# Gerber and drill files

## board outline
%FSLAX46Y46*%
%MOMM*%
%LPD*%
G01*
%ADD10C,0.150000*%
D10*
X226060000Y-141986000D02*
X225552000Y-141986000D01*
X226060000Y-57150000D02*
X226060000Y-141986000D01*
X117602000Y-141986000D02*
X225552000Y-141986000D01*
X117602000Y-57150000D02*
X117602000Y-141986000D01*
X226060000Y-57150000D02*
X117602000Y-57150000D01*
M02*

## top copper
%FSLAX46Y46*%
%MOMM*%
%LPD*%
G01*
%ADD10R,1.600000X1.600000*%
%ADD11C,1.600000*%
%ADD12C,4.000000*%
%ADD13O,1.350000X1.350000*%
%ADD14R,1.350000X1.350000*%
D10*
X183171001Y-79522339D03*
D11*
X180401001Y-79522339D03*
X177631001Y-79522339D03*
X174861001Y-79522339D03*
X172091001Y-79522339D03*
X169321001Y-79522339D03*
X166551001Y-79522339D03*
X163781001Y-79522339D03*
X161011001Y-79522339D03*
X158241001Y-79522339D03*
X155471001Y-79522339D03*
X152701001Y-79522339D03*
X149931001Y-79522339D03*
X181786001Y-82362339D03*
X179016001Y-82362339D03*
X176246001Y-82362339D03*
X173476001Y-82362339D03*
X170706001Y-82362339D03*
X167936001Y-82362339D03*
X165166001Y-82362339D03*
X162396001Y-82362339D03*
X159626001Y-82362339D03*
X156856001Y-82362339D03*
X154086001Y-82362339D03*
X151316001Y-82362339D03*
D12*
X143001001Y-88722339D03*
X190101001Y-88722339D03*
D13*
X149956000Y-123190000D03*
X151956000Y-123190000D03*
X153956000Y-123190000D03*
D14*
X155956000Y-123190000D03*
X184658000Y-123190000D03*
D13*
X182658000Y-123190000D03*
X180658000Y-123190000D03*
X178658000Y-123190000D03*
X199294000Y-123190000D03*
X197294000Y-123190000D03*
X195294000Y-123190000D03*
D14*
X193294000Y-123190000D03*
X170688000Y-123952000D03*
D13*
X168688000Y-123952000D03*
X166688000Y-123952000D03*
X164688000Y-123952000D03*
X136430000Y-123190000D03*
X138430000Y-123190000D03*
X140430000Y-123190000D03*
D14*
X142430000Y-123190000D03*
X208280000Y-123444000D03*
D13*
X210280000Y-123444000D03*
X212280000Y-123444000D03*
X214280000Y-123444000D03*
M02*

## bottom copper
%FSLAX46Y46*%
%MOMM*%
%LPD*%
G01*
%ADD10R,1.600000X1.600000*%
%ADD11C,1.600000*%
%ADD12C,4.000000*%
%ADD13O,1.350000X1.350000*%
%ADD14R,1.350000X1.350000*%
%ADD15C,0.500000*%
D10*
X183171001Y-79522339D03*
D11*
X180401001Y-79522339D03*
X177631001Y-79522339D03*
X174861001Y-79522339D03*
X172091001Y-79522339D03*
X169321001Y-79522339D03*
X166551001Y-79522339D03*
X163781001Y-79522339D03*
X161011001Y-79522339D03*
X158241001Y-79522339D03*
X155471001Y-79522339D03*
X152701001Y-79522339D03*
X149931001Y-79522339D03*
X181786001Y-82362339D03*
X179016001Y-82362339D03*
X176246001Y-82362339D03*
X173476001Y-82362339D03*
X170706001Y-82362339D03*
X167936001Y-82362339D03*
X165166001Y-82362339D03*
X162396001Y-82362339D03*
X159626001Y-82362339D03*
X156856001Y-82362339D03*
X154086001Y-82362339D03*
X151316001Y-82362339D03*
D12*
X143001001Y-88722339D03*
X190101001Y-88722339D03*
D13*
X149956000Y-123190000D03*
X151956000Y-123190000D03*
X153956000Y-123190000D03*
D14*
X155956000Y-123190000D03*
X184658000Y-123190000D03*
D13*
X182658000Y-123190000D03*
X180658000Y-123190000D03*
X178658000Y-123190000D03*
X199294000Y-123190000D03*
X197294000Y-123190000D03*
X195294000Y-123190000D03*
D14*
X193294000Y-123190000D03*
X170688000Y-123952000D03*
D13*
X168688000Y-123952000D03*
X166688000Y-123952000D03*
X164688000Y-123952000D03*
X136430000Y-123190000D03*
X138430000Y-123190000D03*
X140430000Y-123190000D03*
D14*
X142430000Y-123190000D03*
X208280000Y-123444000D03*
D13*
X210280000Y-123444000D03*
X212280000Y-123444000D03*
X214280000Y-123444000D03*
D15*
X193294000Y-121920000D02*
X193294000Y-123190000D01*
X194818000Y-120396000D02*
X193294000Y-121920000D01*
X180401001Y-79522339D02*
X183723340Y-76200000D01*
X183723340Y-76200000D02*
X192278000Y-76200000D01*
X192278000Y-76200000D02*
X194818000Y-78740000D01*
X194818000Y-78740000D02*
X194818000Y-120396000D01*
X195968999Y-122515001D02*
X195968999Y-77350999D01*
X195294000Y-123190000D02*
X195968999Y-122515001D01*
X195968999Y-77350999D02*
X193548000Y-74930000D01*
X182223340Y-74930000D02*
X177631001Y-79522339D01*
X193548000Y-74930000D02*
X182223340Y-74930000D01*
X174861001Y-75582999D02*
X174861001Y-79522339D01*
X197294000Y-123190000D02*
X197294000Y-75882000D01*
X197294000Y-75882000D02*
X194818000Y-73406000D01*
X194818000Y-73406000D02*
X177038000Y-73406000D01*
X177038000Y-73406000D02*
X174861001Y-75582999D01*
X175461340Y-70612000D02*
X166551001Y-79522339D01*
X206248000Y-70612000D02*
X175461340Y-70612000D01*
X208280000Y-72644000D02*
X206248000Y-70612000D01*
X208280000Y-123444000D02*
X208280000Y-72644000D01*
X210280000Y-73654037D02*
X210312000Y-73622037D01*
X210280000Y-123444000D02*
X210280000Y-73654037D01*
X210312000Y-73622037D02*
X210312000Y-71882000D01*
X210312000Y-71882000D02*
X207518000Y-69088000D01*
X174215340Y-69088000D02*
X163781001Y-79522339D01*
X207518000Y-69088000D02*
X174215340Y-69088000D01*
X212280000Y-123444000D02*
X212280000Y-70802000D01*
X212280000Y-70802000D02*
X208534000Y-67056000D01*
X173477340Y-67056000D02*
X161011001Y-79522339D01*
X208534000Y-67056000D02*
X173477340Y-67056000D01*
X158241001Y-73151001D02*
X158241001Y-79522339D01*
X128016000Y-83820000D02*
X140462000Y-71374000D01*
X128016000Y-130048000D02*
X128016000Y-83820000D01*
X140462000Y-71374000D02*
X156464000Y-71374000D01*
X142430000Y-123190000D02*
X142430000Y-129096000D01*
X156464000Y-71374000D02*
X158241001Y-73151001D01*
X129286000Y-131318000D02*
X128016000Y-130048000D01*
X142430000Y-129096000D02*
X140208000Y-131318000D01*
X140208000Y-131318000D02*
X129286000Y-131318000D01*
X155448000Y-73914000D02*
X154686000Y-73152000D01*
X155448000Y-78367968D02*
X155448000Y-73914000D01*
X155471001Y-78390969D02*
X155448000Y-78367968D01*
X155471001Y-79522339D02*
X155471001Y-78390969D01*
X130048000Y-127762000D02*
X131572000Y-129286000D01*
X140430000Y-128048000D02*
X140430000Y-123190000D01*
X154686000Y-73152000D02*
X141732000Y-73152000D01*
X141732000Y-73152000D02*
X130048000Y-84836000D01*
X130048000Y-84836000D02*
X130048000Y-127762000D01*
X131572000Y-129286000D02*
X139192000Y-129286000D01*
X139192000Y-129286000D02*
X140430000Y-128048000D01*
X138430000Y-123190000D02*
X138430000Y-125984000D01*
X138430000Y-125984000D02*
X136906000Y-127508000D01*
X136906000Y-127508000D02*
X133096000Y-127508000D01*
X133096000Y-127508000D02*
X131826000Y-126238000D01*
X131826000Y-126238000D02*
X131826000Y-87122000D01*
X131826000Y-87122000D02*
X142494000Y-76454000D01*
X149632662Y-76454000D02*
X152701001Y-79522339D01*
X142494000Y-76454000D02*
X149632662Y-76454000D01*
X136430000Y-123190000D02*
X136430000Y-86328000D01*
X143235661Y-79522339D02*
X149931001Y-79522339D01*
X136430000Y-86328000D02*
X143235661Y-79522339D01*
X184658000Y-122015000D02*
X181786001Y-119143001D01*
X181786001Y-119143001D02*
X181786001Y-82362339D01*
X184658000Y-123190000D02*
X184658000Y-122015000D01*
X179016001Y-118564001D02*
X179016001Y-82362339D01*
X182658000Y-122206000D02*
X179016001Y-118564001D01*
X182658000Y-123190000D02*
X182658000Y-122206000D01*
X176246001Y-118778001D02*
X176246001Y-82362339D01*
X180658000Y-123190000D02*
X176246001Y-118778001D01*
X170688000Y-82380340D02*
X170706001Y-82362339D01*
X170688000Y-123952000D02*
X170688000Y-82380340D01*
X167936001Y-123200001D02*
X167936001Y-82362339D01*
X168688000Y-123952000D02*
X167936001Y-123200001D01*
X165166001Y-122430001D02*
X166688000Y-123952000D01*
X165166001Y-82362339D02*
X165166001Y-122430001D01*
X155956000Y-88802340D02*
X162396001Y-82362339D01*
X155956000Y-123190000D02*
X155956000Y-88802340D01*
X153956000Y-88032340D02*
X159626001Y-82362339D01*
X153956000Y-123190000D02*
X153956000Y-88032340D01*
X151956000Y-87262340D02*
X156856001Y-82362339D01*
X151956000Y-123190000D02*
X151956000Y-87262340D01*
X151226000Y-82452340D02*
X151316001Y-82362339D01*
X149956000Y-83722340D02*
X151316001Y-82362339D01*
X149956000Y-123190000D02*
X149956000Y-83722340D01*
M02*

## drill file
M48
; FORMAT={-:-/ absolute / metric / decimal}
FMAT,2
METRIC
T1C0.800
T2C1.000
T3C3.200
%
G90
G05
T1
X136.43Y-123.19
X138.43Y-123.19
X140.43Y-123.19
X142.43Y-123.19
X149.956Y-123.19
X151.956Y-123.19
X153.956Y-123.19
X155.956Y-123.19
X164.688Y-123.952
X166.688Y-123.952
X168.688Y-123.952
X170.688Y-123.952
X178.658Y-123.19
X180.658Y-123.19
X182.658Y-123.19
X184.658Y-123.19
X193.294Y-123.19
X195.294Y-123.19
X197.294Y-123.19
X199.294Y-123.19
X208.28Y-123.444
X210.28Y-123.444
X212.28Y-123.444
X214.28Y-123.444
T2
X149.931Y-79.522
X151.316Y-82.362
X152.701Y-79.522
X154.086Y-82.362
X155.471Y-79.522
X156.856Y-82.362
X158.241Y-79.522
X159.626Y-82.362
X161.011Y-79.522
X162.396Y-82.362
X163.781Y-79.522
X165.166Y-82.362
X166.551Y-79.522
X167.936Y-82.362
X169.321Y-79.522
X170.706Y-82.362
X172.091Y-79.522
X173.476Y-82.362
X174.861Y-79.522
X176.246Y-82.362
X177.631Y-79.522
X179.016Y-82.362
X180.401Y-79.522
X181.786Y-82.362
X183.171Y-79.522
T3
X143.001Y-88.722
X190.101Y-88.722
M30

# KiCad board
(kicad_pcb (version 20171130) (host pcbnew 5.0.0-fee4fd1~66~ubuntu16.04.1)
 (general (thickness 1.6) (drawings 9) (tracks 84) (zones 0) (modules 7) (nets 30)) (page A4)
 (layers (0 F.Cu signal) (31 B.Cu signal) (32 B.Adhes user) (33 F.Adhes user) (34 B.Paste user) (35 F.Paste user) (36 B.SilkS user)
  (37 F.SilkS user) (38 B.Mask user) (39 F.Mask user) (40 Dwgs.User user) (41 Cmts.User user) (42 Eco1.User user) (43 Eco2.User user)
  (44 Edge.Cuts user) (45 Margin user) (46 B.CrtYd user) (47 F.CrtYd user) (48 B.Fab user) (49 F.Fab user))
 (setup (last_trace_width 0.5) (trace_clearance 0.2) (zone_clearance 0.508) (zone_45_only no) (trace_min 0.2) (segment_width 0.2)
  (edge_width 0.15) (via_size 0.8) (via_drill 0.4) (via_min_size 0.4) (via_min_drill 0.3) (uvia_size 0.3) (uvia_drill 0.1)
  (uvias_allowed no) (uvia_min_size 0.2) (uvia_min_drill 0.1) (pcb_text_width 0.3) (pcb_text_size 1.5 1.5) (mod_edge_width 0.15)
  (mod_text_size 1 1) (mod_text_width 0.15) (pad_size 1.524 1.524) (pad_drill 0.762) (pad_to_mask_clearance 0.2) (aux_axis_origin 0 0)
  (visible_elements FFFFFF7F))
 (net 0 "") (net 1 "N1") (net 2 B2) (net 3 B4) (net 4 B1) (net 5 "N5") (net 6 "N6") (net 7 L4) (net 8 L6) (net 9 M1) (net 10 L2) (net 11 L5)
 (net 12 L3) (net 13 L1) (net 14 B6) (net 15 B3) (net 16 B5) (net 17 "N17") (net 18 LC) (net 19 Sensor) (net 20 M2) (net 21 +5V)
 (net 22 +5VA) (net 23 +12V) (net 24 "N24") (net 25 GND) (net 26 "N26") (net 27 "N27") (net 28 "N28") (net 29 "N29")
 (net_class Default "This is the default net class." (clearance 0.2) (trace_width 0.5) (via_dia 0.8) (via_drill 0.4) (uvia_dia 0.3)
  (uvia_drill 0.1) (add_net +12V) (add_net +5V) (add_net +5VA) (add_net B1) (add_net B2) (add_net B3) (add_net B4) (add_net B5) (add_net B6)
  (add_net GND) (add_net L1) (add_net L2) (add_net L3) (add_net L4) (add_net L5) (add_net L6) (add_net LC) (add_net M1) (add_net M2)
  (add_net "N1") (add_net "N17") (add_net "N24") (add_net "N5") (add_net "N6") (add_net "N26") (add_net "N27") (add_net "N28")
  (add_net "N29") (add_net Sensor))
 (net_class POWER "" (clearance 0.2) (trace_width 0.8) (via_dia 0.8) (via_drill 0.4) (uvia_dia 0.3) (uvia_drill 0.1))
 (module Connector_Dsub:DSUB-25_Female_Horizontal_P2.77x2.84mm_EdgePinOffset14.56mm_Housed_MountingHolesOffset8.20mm (layer F.Cu)
  (at 183.171001 79.522339)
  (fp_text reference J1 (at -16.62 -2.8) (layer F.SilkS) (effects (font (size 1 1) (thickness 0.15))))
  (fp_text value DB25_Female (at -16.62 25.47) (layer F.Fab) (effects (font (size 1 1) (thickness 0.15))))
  (pad 1 thru_hole rect (at 0 0) (size 1.6 1.6) (drill 1) (layers *.Cu *.Mask) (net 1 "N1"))
  (pad 2 thru_hole circle (at -2.77 0) (size 1.6 1.6) (drill 1) (layers *.Cu *.Mask) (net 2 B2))
  (pad 3 thru_hole circle (at -5.54 0) (size 1.6 1.6) (drill 1) (layers *.Cu *.Mask) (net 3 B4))
  (pad 4 thru_hole circle (at -8.31 0) (size 1.6 1.6) (drill 1) (layers *.Cu *.Mask) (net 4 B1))
  (pad 5 thru_hole circle (at -11.08 0) (size 1.6 1.6) (drill 1) (layers *.Cu *.Mask) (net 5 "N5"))
  (pad 6 thru_hole circle (at -13.85 0) (size 1.6 1.6) (drill 1) (layers *.Cu *.Mask) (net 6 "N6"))
  (pad 7 thru_hole circle (at -16.62 0) (size 1.6 1.6) (drill 1) (layers *.Cu *.Mask) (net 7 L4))
  (pad 8 thru_hole circle (at -19.39 0) (size 1.6 1.6) (drill 1) (layers *.Cu *.Mask) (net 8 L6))
  (pad 9 thru_hole circle (at -22.16 0) (size 1.6 1.6) (drill 1) (layers *.Cu *.Mask) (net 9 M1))
  (pad 10 thru_hole circle (at -24.93 0) (size 1.6 1.6) (drill 1) (layers *.Cu *.Mask) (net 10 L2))
  (pad 11 thru_hole circle (at -27.7 0) (size 1.6 1.6) (drill 1) (layers *.Cu *.Mask) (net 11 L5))
  (pad 12 thru_hole circle (at -30.47 0) (size 1.6 1.6) (drill 1) (layers *.Cu *.Mask) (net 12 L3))
  (pad 13 thru_hole circle (at -33.24 0) (size 1.6 1.6) (drill 1) (layers *.Cu *.Mask) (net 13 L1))
  (pad 14 thru_hole circle (at -1.385 2.84) (size 1.6 1.6) (drill 1) (layers *.Cu *.Mask) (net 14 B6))
  (pad 15 thru_hole circle (at -4.155 2.84) (size 1.6 1.6) (drill 1) (layers *.Cu *.Mask) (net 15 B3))
  (pad 16 thru_hole circle (at -6.925 2.84) (size 1.6 1.6) (drill 1) (layers *.Cu *.Mask) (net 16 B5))
  (pad 17 thru_hole circle (at -9.695 2.84) (size 1.6 1.6) (drill 1) (layers *.Cu *.Mask) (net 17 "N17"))
  (pad 18 thru_hole circle (at -12.465 2.84) (size 1.6 1.6) (drill 1) (layers *.Cu *.Mask) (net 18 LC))
  (pad 19 thru_hole circle (at -15.235 2.84) (size 1.6 1.6) (drill 1) (layers *.Cu *.Mask) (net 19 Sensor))
  (pad 20 thru_hole circle (at -18.005 2.84) (size 1.6 1.6) (drill 1) (layers *.Cu *.Mask) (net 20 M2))
  (pad 21 thru_hole circle (at -20.775 2.84) (size 1.6 1.6) (drill 1) (layers *.Cu *.Mask) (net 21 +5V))
  (pad 22 thru_hole circle (at -23.545 2.84) (size 1.6 1.6) (drill 1) (layers *.Cu *.Mask) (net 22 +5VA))
  (pad 23 thru_hole circle (at -26.315 2.84) (size 1.6 1.6) (drill 1) (layers *.Cu *.Mask) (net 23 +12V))
  (pad 24 thru_hole circle (at -29.085 2.84) (size 1.6 1.6) (drill 1) (layers *.Cu *.Mask) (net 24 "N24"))
  (pad 25 thru_hole circle (at -31.855 2.84) (size 1.6 1.6) (drill 1) (layers *.Cu *.Mask) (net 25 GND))
  (pad 0 thru_hole circle (at -40.17 9.2) (size 4 4) (drill 3.2) (layers *.Cu *.Mask))
  (pad 0 thru_hole circle (at 6.93 9.2) (size 4 4) (drill 3.2) (layers *.Cu *.Mask)))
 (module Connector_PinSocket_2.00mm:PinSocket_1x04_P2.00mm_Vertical (layer F.Cu) (at 155.956 123.19 270)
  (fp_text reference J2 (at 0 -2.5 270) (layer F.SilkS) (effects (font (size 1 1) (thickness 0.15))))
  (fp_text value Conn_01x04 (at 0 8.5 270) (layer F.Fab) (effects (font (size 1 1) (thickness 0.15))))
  (pad 4 thru_hole oval (at 0 6 270) (size 1.35 1.35) (drill 0.8) (layers *.Cu *.Mask) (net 25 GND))
  (pad 3 thru_hole oval (at 0 4 270) (size 1.35 1.35) (drill 0.8) (layers *.Cu *.Mask) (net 23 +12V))
  (pad 2 thru_hole oval (at 0 2 270) (size 1.35 1.35) (drill 0.8) (layers *.Cu *.Mask) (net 22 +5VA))
  (pad 1 thru_hole rect (at 0 0 270) (size 1.35 1.35) (drill 0.8) (layers *.Cu *.Mask) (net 21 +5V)))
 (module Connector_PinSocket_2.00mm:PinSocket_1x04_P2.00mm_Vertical (layer F.Cu) (at 184.658 123.19 270)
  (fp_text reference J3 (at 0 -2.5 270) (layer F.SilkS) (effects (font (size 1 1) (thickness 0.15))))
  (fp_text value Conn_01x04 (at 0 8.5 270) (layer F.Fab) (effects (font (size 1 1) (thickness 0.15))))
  (pad 1 thru_hole rect (at 0 0 270) (size 1.35 1.35) (drill 0.8) (layers *.Cu *.Mask) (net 14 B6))
  (pad 2 thru_hole oval (at 0 2 270) (size 1.35 1.35) (drill 0.8) (layers *.Cu *.Mask) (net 15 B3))
  (pad 3 thru_hole oval (at 0 4 270) (size 1.35 1.35) (drill 0.8) (layers *.Cu *.Mask) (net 16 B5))
  (pad 4 thru_hole oval (at 0 6 270) (size 1.35 1.35) (drill 0.8) (layers *.Cu *.Mask) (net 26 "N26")))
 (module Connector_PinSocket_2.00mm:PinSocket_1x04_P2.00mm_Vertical (layer F.Cu) (at 193.294 123.19 90)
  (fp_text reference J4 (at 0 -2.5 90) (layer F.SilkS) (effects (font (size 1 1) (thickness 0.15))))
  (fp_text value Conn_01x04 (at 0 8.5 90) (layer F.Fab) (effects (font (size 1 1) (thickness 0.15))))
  (pad 4 thru_hole oval (at 0 6 90) (size 1.35 1.35) (drill 0.8) (layers *.Cu *.Mask) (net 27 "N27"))
  (pad 3 thru_hole oval (at 0 4 90) (size 1.35 1.35) (drill 0.8) (layers *.Cu *.Mask) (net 4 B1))
  (pad 2 thru_hole oval (at 0 2 90) (size 1.35 1.35) (drill 0.8) (layers *.Cu *.Mask) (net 3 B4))
  (pad 1 thru_hole rect (at 0 0 90) (size 1.35 1.35) (drill 0.8) (layers *.Cu *.Mask) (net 2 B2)))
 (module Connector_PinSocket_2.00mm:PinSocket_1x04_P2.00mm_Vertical (layer F.Cu) (at 170.688 123.952 270)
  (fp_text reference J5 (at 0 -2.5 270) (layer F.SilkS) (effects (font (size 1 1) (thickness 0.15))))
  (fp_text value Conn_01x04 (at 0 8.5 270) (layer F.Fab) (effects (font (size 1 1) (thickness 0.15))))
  (pad 1 thru_hole rect (at 0 0 270) (size 1.35 1.35) (drill 0.8) (layers *.Cu *.Mask) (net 18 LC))
  (pad 2 thru_hole oval (at 0 2 270) (size 1.35 1.35) (drill 0.8) (layers *.Cu *.Mask) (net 19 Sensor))
  (pad 3 thru_hole oval (at 0 4 270) (size 1.35 1.35) (drill 0.8) (layers *.Cu *.Mask) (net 20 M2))
  (pad 4 thru_hole oval (at 0 6 270) (size 1.35 1.35) (drill 0.8) (layers *.Cu *.Mask) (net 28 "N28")))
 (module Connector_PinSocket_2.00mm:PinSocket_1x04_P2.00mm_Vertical (layer F.Cu) (at 142.43 123.19 270)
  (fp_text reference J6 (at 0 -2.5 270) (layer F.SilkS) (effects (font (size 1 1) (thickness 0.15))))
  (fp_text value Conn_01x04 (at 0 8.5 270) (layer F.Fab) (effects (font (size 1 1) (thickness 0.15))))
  (pad 4 thru_hole oval (at 0 6 270) (size 1.35 1.35) (drill 0.8) (layers *.Cu *.Mask) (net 13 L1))
  (pad 3 thru_hole oval (at 0 4 270) (size 1.35 1.35) (drill 0.8) (layers *.Cu *.Mask) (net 12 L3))
  (pad 2 thru_hole oval (at 0 2 270) (size 1.35 1.35) (drill 0.8) (layers *.Cu *.Mask) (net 11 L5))
  (pad 1 thru_hole rect (at 0 0 270) (size 1.35 1.35) (drill 0.8) (layers *.Cu *.Mask) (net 10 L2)))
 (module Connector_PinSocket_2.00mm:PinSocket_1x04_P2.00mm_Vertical (layer F.Cu) (at 208.28 123.444 90)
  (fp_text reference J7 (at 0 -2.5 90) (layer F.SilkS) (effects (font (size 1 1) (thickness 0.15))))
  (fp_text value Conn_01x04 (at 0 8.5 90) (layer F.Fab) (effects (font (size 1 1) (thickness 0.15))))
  (pad 1 thru_hole rect (at 0 0 90) (size 1.35 1.35) (drill 0.8) (layers *.Cu *.Mask) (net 7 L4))
  (pad 2 thru_hole oval (at 0 2 90) (size 1.35 1.35) (drill 0.8) (layers *.Cu *.Mask) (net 8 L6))
  (pad 3 thru_hole oval (at 0 4 90) (size 1.35 1.35) (drill 0.8) (layers *.Cu *.Mask) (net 9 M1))
  (pad 4 thru_hole oval (at 0 6 90) (size 1.35 1.35) (drill 0.8) (layers *.Cu *.Mask) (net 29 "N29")))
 (gr_line (start 226.06 141.986) (end 225.552 141.986) (layer Edge.Cuts) (width 0.15))
 (gr_line (start 226.06 57.15) (end 226.06 141.986) (layer Edge.Cuts) (width 0.15))
 (gr_line (start 117.602 141.986) (end 225.552 141.986) (layer Edge.Cuts) (width 0.15))
 (gr_line (start 117.602 57.15) (end 117.602 141.986) (layer Edge.Cuts) (width 0.15))
 (gr_line (start 226.06 57.15) (end 117.602 57.15) (layer Edge.Cuts) (width 0.15))
 (segment (start 193.294 121.92) (end 193.294 123.19) (width 0.5) (layer B.Cu) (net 2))
 (segment (start 194.818 120.396) (end 193.294 121.92) (width 0.5) (layer B.Cu) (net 2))
 (segment (start 180.401001 79.522339) (end 183.72334 76.2) (width 0.5) (layer B.Cu) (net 2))
 (segment (start 183.72334 76.2) (end 192.278 76.2) (width 0.5) (layer B.Cu) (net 2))
 (segment (start 192.278 76.2) (end 194.818 78.74) (width 0.5) (layer B.Cu) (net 2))
 (segment (start 194.818 78.74) (end 194.818 120.396) (width 0.5) (layer B.Cu) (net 2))
 (segment (start 195.968999 122.515001) (end 195.968999 77.350999) (width 0.5) (layer B.Cu) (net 3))
 (segment (start 195.294 123.19) (end 195.968999 122.515001) (width 0.5) (layer B.Cu) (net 3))
 (segment (start 195.968999 77.350999) (end 193.548 74.93) (width 0.5) (layer B.Cu) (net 3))
 (segment (start 182.22334 74.93) (end 177.631001 79.522339) (width 0.5) (layer B.Cu) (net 3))
 (segment (start 193.548 74.93) (end 182.22334 74.93) (width 0.5) (layer B.Cu) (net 3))
 (segment (start 174.861001 75.582999) (end 174.861001 79.522339) (width 0.5) (layer B.Cu) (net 4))
 (segment (start 197.294 123.19) (end 197.294 75.882) (width 0.5) (layer B.Cu) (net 4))
 (segment (start 197.294 75.882) (end 194.818 73.406) (width 0.5) (layer B.Cu) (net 4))
 (segment (start 194.818 73.406) (end 177.038 73.406) (width 0.5) (layer B.Cu) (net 4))
 (segment (start 177.038 73.406) (end 174.861001 75.582999) (width 0.5) (layer B.Cu) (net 4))
 (segment (start 175.46134 70.612) (end 166.551001 79.522339) (width 0.5) (layer B.Cu) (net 7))
 (segment (start 206.248 70.612) (end 175.46134 70.612) (width 0.5) (layer B.Cu) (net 7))
 (segment (start 208.28 72.644) (end 206.248 70.612) (width 0.5) (layer B.Cu) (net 7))
 (segment (start 208.28 123.444) (end 208.28 72.644) (width 0.5) (layer B.Cu) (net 7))
 (segment (start 210.28 73.654037) (end 210.312 73.622037) (width 0.5) (layer B.Cu) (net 8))
 (segment (start 210.28 123.444) (end 210.28 73.654037) (width 0.5) (layer B.Cu) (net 8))
 (segment (start 210.312 73.622037) (end 210.312 71.882) (width 0.5) (layer B.Cu) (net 8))
 (segment (start 210.312 71.882) (end 207.518 69.088) (width 0.5) (layer B.Cu) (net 8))
 (segment (start 174.21534 69.088) (end 163.781001 79.522339) (width 0.5) (layer B.Cu) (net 8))
 (segment (start 207.518 69.088) (end 174.21534 69.088) (width 0.5) (layer B.Cu) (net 8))
 (segment (start 212.28 123.444) (end 212.28 70.802) (width 0.5) (layer B.Cu) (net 9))
 (segment (start 212.28 70.802) (end 208.534 67.056) (width 0.5) (layer B.Cu) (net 9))
 (segment (start 173.47734 67.056) (end 161.011001 79.522339) (width 0.5) (layer B.Cu) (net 9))
 (segment (start 208.534 67.056) (end 173.47734 67.056) (width 0.5) (layer B.Cu) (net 9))
 (segment (start 158.241001 73.151001) (end 158.241001 79.522339) (width 0.5) (layer B.Cu) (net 10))
 (segment (start 128.016 83.82) (end 140.462 71.374) (width 0.5) (layer B.Cu) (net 10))
 (segment (start 128.016 130.048) (end 128.016 83.82) (width 0.5) (layer B.Cu) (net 10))
 (segment (start 140.462 71.374) (end 156.464 71.374) (width 0.5) (layer B.Cu) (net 10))
 (segment (start 142.43 123.19) (end 142.43 129.096) (width 0.5) (layer B.Cu) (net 10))
 (segment (start 156.464 71.374) (end 158.241001 73.151001) (width 0.5) (layer B.Cu) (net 10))
 (segment (start 129.286 131.318) (end 128.016 130.048) (width 0.5) (layer B.Cu) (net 10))
 (segment (start 142.43 129.096) (end 140.208 131.318) (width 0.5) (layer B.Cu) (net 10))
 (segment (start 140.208 131.318) (end 129.286 131.318) (width 0.5) (layer B.Cu) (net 10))
 (segment (start 155.448 73.914) (end 154.686 73.152) (width 0.5) (layer B.Cu) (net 11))
 (segment (start 155.448 78.367968) (end 155.448 73.914) (width 0.5) (layer B.Cu) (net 11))
 (segment (start 155.471001 78.390969) (end 155.448 78.367968) (width 0.5) (layer B.Cu) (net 11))
 (segment (start 155.471001 79.522339) (end 155.471001 78.390969) (width 0.5) (layer B.Cu) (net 11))
 (segment (start 130.048 127.762) (end 131.572 129.286) (width 0.5) (layer B.Cu) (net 11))
 (segment (start 140.43 128.048) (end 140.43 123.19) (width 0.5) (layer B.Cu) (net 11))
 (segment (start 154.686 73.152) (end 141.732 73.152) (width 0.5) (layer B.Cu) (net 11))
 (segment (start 141.732 73.152) (end 130.048 84.836) (width 0.5) (layer B.Cu) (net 11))
 (segment (start 130.048 84.836) (end 130.048 127.762) (width 0.5) (layer B.Cu) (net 11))
 (segment (start 131.572 129.286) (end 139.192 129.286) (width 0.5) (layer B.Cu) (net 11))
 (segment (start 139.192 129.286) (end 140.43 128.048) (width 0.5) (layer B.Cu) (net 11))
 (segment (start 138.43 123.19) (end 138.43 125.984) (width 0.5) (layer B.Cu) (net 12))
 (segment (start 138.43 125.984) (end 136.906 127.508) (width 0.5) (layer B.Cu) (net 12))
 (segment (start 136.906 127.508) (end 133.096 127.508) (width 0.5) (layer B.Cu) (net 12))
 (segment (start 133.096 127.508) (end 131.826 126.238) (width 0.5) (layer B.Cu) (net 12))
 (segment (start 131.826 126.238) (end 131.826 87.122) (width 0.5) (layer B.Cu) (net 12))
 (segment (start 131.826 87.122) (end 142.494 76.454) (width 0.5) (layer B.Cu) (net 12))
 (segment (start 149.632662 76.454) (end 152.701001 79.522339) (width 0.5) (layer B.Cu) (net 12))
 (segment (start 142.494 76.454) (end 149.632662 76.454) (width 0.5) (layer B.Cu) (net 12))
 (segment (start 136.43 123.19) (end 136.43 86.328) (width 0.5) (layer B.Cu) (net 13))
 (segment (start 143.235661 79.522339) (end 149.931001 79.522339) (width 0.5) (layer B.Cu) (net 13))
 (segment (start 136.43 86.328) (end 143.235661 79.522339) (width 0.5) (layer B.Cu) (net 13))
 (segment (start 184.658 122.015) (end 181.786001 119.143001) (width 0.5) (layer B.Cu) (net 14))
 (segment (start 181.786001 119.143001) (end 181.786001 82.362339) (width 0.5) (layer B.Cu) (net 14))
 (segment (start 184.658 123.19) (end 184.658 122.015) (width 0.5) (layer B.Cu) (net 14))
 (segment (start 179.016001 118.564001) (end 179.016001 82.362339) (width 0.5) (layer B.Cu) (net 15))
 (segment (start 182.658 122.206) (end 179.016001 118.564001) (width 0.5) (layer B.Cu) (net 15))
 (segment (start 182.658 123.19) (end 182.658 122.206) (width 0.5) (layer B.Cu) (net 15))
 (segment (start 176.246001 118.778001) (end 176.246001 82.362339) (width 0.5) (layer B.Cu) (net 16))
 (segment (start 180.658 123.19) (end 176.246001 118.778001) (width 0.5) (layer B.Cu) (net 16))
 (segment (start 170.688 82.38034) (end 170.706001 82.362339) (width 0.5) (layer B.Cu) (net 18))
 (segment (start 170.688 123.952) (end 170.688 82.38034) (width 0.5) (layer B.Cu) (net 18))
 (segment (start 167.936001 123.200001) (end 167.936001 82.362339) (width 0.5) (layer B.Cu) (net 19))
 (segment (start 168.688 123.952) (end 167.936001 123.200001) (width 0.5) (layer B.Cu) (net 19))
 (segment (start 165.166001 122.430001) (end 166.688 123.952) (width 0.5) (layer B.Cu) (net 20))
 (segment (start 165.166001 82.362339) (end 165.166001 122.430001) (width 0.5) (layer B.Cu) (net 20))
 (segment (start 155.956 88.80234) (end 162.396001 82.362339) (width 0.5) (layer B.Cu) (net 21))
 (segment (start 155.956 123.19) (end 155.956 88.80234) (width 0.5) (layer B.Cu) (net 21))
 (segment (start 153.956 88.03234) (end 159.626001 82.362339) (width 0.5) (layer B.Cu) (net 22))
 (segment (start 153.956 123.19) (end 153.956 88.03234) (width 0.5) (layer B.Cu) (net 22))
 (segment (start 151.956 87.26234) (end 156.856001 82.362339) (width 0.5) (layer B.Cu) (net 23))
 (segment (start 151.956 123.19) (end 151.956 87.26234) (width 0.5) (layer B.Cu) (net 23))
 (segment (start 151.226 82.45234) (end 151.316001 82.362339) (width 0.5) (layer B.Cu) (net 25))
 (segment (start 149.956 83.72234) (end 151.316001 82.362339) (width 0.5) (layer B.Cu) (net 25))
 (segment (start 149.956 123.19) (end 149.956 83.72234) (width 0.5) (layer B.Cu) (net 25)))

